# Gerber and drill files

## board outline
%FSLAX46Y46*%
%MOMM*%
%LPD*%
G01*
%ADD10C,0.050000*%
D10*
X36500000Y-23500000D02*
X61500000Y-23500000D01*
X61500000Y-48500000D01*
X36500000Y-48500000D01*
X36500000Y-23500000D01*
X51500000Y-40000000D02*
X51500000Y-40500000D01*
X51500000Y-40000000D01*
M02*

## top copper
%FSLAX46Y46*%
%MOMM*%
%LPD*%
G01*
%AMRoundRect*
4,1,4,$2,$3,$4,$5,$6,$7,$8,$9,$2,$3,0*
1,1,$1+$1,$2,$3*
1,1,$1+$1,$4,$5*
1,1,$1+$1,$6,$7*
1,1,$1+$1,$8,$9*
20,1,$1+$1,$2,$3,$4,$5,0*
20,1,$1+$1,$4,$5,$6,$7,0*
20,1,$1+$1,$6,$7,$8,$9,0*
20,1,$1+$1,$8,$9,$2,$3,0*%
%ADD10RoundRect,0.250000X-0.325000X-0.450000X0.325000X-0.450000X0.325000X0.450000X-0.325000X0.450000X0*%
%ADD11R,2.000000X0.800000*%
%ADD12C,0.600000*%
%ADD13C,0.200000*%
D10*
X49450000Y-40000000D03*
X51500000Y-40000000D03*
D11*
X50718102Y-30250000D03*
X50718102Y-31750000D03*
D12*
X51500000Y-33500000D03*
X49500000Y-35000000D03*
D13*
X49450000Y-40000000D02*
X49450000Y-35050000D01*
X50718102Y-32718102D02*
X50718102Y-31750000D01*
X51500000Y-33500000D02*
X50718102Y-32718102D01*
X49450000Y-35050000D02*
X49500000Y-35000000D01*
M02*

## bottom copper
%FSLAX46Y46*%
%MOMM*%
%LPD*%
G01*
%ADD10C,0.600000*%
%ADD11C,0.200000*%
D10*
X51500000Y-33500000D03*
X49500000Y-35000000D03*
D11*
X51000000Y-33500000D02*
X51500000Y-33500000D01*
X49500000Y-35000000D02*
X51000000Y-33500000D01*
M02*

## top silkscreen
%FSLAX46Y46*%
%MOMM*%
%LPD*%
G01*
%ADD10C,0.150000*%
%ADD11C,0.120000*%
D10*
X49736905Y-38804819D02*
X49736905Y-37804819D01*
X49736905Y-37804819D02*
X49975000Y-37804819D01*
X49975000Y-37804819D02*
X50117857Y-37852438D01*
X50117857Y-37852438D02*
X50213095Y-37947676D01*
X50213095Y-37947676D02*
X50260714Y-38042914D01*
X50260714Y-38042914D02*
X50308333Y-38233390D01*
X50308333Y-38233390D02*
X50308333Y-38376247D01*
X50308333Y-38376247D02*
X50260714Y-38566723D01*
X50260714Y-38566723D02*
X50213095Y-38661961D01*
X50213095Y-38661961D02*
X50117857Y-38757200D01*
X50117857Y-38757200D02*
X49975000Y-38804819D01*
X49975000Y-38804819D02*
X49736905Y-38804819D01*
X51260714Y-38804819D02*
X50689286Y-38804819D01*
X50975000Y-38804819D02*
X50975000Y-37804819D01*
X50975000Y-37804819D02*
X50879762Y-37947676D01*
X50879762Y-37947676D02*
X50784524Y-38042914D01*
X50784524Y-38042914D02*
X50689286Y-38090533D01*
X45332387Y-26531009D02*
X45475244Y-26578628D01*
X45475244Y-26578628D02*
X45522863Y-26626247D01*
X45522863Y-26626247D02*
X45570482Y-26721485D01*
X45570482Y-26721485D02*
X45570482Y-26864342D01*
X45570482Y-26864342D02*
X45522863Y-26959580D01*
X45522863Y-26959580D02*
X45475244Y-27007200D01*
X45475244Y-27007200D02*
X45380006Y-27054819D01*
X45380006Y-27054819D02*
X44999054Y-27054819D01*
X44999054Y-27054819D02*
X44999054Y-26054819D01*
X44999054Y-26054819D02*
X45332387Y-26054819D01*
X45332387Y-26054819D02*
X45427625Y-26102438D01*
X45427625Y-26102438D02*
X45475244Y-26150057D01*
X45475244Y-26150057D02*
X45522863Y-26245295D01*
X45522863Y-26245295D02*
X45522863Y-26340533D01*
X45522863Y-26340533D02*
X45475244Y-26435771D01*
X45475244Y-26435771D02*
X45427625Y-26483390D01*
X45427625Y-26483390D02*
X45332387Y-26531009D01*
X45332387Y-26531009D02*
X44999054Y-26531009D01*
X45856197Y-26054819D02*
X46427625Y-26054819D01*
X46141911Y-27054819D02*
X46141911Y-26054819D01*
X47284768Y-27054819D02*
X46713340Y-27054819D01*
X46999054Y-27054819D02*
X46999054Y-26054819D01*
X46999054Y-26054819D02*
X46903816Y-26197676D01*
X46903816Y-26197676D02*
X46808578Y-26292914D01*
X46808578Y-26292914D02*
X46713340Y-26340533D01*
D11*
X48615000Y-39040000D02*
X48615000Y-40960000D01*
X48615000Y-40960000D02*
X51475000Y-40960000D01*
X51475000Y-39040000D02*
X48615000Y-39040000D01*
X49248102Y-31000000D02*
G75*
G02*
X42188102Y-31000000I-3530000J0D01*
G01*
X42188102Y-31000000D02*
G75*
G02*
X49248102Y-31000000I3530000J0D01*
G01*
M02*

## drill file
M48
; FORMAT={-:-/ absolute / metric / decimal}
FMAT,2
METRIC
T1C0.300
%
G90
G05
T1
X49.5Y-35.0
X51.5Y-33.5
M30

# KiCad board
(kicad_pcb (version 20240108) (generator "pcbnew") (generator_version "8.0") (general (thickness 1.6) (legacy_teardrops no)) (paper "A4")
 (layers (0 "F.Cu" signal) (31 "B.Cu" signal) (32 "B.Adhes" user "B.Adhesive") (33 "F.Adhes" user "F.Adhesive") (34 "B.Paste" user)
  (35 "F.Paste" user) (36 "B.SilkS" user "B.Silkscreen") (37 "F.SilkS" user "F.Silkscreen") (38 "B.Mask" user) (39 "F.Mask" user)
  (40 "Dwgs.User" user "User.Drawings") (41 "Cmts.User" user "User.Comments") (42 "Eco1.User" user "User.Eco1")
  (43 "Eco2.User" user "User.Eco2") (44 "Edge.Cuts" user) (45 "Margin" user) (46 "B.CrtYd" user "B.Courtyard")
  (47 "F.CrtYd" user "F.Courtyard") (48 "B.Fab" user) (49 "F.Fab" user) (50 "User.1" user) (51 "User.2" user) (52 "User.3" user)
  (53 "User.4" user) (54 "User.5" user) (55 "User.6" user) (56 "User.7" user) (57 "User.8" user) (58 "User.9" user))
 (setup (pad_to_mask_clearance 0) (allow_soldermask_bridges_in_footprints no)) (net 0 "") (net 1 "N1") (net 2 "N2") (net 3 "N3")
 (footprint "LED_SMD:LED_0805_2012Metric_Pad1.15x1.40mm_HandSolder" (layer "F.Cu") (at 50.475 40)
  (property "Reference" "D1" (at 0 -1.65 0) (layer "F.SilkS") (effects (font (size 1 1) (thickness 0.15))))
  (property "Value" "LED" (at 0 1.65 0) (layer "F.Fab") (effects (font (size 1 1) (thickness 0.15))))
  (fp_line (start -1.86 -0.96) (end -1.86 0.96) (stroke (width 0.12) (type solid)) (layer "F.SilkS"))
  (fp_line (start -1.86 0.96) (end 1 0.96) (stroke (width 0.12) (type solid)) (layer "F.SilkS"))
  (fp_line (start 1 -0.96) (end -1.86 -0.96) (stroke (width 0.12) (type solid)) (layer "F.SilkS"))
  (pad "1" smd roundrect (at -1.025 0) (size 1.15 1.4) (layers "F.Cu" "F.Paste" "F.Mask") (roundrect_rratio 0.217391) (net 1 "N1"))
  (pad "2" smd roundrect (at 1.025 0) (size 1.15 1.4) (layers "F.Cu" "F.Paste" "F.Mask") (roundrect_rratio 0.217391) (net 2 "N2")))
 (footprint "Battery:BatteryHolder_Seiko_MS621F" (layer "F.Cu") (at 50.718102 31)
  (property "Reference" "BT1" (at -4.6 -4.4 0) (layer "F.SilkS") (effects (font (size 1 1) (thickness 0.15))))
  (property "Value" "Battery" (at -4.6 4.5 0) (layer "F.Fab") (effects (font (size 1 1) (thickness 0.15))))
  (fp_circle (center -5 0) (end -1.47 0) (stroke (width 0.12) (type solid)) (fill none) (layer "F.SilkS"))
  (pad "1" smd rect (at 0 -0.75) (size 2 0.8) (layers "F.Cu" "F.Paste" "F.Mask") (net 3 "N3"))
  (pad "2" smd rect (at 0 0.75) (size 2 0.8) (layers "F.Cu" "F.Paste" "F.Mask") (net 1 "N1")))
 (gr_rect (start 36.5 23.5) (end 61.5 48.5) (stroke (width 0.05) (type default)) (fill none) (layer "Edge.Cuts"))
 (gr_rect (start 51.5 40) (end 51.5 40.5) (stroke (width 0.05) (type default)) (fill none) (layer "Edge.Cuts"))
 (segment (start 49.45 40) (end 49.45 35.05) (width 0.2) (layer "F.Cu") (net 1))
 (segment (start 50.718102 32.718102) (end 50.718102 31.75) (width 0.2) (layer "F.Cu") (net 1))
 (segment (start 51.5 33.5) (end 50.718102 32.718102) (width 0.2) (layer "F.Cu") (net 1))
 (segment (start 49.45 35.05) (end 49.5 35) (width 0.2) (layer "F.Cu") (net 1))
 (via (at 51.5 33.5) (size 0.6) (drill 0.3) (layers "F.Cu" "B.Cu") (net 1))
 (via (at 49.5 35) (size 0.6) (drill 0.3) (layers "F.Cu" "B.Cu") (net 1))
 (segment (start 51 33.5) (end 51.5 33.5) (width 0.2) (layer "B.Cu") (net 1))
 (segment (start 49.5 35) (end 51 33.5) (width 0.2) (layer "B.Cu") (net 1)))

